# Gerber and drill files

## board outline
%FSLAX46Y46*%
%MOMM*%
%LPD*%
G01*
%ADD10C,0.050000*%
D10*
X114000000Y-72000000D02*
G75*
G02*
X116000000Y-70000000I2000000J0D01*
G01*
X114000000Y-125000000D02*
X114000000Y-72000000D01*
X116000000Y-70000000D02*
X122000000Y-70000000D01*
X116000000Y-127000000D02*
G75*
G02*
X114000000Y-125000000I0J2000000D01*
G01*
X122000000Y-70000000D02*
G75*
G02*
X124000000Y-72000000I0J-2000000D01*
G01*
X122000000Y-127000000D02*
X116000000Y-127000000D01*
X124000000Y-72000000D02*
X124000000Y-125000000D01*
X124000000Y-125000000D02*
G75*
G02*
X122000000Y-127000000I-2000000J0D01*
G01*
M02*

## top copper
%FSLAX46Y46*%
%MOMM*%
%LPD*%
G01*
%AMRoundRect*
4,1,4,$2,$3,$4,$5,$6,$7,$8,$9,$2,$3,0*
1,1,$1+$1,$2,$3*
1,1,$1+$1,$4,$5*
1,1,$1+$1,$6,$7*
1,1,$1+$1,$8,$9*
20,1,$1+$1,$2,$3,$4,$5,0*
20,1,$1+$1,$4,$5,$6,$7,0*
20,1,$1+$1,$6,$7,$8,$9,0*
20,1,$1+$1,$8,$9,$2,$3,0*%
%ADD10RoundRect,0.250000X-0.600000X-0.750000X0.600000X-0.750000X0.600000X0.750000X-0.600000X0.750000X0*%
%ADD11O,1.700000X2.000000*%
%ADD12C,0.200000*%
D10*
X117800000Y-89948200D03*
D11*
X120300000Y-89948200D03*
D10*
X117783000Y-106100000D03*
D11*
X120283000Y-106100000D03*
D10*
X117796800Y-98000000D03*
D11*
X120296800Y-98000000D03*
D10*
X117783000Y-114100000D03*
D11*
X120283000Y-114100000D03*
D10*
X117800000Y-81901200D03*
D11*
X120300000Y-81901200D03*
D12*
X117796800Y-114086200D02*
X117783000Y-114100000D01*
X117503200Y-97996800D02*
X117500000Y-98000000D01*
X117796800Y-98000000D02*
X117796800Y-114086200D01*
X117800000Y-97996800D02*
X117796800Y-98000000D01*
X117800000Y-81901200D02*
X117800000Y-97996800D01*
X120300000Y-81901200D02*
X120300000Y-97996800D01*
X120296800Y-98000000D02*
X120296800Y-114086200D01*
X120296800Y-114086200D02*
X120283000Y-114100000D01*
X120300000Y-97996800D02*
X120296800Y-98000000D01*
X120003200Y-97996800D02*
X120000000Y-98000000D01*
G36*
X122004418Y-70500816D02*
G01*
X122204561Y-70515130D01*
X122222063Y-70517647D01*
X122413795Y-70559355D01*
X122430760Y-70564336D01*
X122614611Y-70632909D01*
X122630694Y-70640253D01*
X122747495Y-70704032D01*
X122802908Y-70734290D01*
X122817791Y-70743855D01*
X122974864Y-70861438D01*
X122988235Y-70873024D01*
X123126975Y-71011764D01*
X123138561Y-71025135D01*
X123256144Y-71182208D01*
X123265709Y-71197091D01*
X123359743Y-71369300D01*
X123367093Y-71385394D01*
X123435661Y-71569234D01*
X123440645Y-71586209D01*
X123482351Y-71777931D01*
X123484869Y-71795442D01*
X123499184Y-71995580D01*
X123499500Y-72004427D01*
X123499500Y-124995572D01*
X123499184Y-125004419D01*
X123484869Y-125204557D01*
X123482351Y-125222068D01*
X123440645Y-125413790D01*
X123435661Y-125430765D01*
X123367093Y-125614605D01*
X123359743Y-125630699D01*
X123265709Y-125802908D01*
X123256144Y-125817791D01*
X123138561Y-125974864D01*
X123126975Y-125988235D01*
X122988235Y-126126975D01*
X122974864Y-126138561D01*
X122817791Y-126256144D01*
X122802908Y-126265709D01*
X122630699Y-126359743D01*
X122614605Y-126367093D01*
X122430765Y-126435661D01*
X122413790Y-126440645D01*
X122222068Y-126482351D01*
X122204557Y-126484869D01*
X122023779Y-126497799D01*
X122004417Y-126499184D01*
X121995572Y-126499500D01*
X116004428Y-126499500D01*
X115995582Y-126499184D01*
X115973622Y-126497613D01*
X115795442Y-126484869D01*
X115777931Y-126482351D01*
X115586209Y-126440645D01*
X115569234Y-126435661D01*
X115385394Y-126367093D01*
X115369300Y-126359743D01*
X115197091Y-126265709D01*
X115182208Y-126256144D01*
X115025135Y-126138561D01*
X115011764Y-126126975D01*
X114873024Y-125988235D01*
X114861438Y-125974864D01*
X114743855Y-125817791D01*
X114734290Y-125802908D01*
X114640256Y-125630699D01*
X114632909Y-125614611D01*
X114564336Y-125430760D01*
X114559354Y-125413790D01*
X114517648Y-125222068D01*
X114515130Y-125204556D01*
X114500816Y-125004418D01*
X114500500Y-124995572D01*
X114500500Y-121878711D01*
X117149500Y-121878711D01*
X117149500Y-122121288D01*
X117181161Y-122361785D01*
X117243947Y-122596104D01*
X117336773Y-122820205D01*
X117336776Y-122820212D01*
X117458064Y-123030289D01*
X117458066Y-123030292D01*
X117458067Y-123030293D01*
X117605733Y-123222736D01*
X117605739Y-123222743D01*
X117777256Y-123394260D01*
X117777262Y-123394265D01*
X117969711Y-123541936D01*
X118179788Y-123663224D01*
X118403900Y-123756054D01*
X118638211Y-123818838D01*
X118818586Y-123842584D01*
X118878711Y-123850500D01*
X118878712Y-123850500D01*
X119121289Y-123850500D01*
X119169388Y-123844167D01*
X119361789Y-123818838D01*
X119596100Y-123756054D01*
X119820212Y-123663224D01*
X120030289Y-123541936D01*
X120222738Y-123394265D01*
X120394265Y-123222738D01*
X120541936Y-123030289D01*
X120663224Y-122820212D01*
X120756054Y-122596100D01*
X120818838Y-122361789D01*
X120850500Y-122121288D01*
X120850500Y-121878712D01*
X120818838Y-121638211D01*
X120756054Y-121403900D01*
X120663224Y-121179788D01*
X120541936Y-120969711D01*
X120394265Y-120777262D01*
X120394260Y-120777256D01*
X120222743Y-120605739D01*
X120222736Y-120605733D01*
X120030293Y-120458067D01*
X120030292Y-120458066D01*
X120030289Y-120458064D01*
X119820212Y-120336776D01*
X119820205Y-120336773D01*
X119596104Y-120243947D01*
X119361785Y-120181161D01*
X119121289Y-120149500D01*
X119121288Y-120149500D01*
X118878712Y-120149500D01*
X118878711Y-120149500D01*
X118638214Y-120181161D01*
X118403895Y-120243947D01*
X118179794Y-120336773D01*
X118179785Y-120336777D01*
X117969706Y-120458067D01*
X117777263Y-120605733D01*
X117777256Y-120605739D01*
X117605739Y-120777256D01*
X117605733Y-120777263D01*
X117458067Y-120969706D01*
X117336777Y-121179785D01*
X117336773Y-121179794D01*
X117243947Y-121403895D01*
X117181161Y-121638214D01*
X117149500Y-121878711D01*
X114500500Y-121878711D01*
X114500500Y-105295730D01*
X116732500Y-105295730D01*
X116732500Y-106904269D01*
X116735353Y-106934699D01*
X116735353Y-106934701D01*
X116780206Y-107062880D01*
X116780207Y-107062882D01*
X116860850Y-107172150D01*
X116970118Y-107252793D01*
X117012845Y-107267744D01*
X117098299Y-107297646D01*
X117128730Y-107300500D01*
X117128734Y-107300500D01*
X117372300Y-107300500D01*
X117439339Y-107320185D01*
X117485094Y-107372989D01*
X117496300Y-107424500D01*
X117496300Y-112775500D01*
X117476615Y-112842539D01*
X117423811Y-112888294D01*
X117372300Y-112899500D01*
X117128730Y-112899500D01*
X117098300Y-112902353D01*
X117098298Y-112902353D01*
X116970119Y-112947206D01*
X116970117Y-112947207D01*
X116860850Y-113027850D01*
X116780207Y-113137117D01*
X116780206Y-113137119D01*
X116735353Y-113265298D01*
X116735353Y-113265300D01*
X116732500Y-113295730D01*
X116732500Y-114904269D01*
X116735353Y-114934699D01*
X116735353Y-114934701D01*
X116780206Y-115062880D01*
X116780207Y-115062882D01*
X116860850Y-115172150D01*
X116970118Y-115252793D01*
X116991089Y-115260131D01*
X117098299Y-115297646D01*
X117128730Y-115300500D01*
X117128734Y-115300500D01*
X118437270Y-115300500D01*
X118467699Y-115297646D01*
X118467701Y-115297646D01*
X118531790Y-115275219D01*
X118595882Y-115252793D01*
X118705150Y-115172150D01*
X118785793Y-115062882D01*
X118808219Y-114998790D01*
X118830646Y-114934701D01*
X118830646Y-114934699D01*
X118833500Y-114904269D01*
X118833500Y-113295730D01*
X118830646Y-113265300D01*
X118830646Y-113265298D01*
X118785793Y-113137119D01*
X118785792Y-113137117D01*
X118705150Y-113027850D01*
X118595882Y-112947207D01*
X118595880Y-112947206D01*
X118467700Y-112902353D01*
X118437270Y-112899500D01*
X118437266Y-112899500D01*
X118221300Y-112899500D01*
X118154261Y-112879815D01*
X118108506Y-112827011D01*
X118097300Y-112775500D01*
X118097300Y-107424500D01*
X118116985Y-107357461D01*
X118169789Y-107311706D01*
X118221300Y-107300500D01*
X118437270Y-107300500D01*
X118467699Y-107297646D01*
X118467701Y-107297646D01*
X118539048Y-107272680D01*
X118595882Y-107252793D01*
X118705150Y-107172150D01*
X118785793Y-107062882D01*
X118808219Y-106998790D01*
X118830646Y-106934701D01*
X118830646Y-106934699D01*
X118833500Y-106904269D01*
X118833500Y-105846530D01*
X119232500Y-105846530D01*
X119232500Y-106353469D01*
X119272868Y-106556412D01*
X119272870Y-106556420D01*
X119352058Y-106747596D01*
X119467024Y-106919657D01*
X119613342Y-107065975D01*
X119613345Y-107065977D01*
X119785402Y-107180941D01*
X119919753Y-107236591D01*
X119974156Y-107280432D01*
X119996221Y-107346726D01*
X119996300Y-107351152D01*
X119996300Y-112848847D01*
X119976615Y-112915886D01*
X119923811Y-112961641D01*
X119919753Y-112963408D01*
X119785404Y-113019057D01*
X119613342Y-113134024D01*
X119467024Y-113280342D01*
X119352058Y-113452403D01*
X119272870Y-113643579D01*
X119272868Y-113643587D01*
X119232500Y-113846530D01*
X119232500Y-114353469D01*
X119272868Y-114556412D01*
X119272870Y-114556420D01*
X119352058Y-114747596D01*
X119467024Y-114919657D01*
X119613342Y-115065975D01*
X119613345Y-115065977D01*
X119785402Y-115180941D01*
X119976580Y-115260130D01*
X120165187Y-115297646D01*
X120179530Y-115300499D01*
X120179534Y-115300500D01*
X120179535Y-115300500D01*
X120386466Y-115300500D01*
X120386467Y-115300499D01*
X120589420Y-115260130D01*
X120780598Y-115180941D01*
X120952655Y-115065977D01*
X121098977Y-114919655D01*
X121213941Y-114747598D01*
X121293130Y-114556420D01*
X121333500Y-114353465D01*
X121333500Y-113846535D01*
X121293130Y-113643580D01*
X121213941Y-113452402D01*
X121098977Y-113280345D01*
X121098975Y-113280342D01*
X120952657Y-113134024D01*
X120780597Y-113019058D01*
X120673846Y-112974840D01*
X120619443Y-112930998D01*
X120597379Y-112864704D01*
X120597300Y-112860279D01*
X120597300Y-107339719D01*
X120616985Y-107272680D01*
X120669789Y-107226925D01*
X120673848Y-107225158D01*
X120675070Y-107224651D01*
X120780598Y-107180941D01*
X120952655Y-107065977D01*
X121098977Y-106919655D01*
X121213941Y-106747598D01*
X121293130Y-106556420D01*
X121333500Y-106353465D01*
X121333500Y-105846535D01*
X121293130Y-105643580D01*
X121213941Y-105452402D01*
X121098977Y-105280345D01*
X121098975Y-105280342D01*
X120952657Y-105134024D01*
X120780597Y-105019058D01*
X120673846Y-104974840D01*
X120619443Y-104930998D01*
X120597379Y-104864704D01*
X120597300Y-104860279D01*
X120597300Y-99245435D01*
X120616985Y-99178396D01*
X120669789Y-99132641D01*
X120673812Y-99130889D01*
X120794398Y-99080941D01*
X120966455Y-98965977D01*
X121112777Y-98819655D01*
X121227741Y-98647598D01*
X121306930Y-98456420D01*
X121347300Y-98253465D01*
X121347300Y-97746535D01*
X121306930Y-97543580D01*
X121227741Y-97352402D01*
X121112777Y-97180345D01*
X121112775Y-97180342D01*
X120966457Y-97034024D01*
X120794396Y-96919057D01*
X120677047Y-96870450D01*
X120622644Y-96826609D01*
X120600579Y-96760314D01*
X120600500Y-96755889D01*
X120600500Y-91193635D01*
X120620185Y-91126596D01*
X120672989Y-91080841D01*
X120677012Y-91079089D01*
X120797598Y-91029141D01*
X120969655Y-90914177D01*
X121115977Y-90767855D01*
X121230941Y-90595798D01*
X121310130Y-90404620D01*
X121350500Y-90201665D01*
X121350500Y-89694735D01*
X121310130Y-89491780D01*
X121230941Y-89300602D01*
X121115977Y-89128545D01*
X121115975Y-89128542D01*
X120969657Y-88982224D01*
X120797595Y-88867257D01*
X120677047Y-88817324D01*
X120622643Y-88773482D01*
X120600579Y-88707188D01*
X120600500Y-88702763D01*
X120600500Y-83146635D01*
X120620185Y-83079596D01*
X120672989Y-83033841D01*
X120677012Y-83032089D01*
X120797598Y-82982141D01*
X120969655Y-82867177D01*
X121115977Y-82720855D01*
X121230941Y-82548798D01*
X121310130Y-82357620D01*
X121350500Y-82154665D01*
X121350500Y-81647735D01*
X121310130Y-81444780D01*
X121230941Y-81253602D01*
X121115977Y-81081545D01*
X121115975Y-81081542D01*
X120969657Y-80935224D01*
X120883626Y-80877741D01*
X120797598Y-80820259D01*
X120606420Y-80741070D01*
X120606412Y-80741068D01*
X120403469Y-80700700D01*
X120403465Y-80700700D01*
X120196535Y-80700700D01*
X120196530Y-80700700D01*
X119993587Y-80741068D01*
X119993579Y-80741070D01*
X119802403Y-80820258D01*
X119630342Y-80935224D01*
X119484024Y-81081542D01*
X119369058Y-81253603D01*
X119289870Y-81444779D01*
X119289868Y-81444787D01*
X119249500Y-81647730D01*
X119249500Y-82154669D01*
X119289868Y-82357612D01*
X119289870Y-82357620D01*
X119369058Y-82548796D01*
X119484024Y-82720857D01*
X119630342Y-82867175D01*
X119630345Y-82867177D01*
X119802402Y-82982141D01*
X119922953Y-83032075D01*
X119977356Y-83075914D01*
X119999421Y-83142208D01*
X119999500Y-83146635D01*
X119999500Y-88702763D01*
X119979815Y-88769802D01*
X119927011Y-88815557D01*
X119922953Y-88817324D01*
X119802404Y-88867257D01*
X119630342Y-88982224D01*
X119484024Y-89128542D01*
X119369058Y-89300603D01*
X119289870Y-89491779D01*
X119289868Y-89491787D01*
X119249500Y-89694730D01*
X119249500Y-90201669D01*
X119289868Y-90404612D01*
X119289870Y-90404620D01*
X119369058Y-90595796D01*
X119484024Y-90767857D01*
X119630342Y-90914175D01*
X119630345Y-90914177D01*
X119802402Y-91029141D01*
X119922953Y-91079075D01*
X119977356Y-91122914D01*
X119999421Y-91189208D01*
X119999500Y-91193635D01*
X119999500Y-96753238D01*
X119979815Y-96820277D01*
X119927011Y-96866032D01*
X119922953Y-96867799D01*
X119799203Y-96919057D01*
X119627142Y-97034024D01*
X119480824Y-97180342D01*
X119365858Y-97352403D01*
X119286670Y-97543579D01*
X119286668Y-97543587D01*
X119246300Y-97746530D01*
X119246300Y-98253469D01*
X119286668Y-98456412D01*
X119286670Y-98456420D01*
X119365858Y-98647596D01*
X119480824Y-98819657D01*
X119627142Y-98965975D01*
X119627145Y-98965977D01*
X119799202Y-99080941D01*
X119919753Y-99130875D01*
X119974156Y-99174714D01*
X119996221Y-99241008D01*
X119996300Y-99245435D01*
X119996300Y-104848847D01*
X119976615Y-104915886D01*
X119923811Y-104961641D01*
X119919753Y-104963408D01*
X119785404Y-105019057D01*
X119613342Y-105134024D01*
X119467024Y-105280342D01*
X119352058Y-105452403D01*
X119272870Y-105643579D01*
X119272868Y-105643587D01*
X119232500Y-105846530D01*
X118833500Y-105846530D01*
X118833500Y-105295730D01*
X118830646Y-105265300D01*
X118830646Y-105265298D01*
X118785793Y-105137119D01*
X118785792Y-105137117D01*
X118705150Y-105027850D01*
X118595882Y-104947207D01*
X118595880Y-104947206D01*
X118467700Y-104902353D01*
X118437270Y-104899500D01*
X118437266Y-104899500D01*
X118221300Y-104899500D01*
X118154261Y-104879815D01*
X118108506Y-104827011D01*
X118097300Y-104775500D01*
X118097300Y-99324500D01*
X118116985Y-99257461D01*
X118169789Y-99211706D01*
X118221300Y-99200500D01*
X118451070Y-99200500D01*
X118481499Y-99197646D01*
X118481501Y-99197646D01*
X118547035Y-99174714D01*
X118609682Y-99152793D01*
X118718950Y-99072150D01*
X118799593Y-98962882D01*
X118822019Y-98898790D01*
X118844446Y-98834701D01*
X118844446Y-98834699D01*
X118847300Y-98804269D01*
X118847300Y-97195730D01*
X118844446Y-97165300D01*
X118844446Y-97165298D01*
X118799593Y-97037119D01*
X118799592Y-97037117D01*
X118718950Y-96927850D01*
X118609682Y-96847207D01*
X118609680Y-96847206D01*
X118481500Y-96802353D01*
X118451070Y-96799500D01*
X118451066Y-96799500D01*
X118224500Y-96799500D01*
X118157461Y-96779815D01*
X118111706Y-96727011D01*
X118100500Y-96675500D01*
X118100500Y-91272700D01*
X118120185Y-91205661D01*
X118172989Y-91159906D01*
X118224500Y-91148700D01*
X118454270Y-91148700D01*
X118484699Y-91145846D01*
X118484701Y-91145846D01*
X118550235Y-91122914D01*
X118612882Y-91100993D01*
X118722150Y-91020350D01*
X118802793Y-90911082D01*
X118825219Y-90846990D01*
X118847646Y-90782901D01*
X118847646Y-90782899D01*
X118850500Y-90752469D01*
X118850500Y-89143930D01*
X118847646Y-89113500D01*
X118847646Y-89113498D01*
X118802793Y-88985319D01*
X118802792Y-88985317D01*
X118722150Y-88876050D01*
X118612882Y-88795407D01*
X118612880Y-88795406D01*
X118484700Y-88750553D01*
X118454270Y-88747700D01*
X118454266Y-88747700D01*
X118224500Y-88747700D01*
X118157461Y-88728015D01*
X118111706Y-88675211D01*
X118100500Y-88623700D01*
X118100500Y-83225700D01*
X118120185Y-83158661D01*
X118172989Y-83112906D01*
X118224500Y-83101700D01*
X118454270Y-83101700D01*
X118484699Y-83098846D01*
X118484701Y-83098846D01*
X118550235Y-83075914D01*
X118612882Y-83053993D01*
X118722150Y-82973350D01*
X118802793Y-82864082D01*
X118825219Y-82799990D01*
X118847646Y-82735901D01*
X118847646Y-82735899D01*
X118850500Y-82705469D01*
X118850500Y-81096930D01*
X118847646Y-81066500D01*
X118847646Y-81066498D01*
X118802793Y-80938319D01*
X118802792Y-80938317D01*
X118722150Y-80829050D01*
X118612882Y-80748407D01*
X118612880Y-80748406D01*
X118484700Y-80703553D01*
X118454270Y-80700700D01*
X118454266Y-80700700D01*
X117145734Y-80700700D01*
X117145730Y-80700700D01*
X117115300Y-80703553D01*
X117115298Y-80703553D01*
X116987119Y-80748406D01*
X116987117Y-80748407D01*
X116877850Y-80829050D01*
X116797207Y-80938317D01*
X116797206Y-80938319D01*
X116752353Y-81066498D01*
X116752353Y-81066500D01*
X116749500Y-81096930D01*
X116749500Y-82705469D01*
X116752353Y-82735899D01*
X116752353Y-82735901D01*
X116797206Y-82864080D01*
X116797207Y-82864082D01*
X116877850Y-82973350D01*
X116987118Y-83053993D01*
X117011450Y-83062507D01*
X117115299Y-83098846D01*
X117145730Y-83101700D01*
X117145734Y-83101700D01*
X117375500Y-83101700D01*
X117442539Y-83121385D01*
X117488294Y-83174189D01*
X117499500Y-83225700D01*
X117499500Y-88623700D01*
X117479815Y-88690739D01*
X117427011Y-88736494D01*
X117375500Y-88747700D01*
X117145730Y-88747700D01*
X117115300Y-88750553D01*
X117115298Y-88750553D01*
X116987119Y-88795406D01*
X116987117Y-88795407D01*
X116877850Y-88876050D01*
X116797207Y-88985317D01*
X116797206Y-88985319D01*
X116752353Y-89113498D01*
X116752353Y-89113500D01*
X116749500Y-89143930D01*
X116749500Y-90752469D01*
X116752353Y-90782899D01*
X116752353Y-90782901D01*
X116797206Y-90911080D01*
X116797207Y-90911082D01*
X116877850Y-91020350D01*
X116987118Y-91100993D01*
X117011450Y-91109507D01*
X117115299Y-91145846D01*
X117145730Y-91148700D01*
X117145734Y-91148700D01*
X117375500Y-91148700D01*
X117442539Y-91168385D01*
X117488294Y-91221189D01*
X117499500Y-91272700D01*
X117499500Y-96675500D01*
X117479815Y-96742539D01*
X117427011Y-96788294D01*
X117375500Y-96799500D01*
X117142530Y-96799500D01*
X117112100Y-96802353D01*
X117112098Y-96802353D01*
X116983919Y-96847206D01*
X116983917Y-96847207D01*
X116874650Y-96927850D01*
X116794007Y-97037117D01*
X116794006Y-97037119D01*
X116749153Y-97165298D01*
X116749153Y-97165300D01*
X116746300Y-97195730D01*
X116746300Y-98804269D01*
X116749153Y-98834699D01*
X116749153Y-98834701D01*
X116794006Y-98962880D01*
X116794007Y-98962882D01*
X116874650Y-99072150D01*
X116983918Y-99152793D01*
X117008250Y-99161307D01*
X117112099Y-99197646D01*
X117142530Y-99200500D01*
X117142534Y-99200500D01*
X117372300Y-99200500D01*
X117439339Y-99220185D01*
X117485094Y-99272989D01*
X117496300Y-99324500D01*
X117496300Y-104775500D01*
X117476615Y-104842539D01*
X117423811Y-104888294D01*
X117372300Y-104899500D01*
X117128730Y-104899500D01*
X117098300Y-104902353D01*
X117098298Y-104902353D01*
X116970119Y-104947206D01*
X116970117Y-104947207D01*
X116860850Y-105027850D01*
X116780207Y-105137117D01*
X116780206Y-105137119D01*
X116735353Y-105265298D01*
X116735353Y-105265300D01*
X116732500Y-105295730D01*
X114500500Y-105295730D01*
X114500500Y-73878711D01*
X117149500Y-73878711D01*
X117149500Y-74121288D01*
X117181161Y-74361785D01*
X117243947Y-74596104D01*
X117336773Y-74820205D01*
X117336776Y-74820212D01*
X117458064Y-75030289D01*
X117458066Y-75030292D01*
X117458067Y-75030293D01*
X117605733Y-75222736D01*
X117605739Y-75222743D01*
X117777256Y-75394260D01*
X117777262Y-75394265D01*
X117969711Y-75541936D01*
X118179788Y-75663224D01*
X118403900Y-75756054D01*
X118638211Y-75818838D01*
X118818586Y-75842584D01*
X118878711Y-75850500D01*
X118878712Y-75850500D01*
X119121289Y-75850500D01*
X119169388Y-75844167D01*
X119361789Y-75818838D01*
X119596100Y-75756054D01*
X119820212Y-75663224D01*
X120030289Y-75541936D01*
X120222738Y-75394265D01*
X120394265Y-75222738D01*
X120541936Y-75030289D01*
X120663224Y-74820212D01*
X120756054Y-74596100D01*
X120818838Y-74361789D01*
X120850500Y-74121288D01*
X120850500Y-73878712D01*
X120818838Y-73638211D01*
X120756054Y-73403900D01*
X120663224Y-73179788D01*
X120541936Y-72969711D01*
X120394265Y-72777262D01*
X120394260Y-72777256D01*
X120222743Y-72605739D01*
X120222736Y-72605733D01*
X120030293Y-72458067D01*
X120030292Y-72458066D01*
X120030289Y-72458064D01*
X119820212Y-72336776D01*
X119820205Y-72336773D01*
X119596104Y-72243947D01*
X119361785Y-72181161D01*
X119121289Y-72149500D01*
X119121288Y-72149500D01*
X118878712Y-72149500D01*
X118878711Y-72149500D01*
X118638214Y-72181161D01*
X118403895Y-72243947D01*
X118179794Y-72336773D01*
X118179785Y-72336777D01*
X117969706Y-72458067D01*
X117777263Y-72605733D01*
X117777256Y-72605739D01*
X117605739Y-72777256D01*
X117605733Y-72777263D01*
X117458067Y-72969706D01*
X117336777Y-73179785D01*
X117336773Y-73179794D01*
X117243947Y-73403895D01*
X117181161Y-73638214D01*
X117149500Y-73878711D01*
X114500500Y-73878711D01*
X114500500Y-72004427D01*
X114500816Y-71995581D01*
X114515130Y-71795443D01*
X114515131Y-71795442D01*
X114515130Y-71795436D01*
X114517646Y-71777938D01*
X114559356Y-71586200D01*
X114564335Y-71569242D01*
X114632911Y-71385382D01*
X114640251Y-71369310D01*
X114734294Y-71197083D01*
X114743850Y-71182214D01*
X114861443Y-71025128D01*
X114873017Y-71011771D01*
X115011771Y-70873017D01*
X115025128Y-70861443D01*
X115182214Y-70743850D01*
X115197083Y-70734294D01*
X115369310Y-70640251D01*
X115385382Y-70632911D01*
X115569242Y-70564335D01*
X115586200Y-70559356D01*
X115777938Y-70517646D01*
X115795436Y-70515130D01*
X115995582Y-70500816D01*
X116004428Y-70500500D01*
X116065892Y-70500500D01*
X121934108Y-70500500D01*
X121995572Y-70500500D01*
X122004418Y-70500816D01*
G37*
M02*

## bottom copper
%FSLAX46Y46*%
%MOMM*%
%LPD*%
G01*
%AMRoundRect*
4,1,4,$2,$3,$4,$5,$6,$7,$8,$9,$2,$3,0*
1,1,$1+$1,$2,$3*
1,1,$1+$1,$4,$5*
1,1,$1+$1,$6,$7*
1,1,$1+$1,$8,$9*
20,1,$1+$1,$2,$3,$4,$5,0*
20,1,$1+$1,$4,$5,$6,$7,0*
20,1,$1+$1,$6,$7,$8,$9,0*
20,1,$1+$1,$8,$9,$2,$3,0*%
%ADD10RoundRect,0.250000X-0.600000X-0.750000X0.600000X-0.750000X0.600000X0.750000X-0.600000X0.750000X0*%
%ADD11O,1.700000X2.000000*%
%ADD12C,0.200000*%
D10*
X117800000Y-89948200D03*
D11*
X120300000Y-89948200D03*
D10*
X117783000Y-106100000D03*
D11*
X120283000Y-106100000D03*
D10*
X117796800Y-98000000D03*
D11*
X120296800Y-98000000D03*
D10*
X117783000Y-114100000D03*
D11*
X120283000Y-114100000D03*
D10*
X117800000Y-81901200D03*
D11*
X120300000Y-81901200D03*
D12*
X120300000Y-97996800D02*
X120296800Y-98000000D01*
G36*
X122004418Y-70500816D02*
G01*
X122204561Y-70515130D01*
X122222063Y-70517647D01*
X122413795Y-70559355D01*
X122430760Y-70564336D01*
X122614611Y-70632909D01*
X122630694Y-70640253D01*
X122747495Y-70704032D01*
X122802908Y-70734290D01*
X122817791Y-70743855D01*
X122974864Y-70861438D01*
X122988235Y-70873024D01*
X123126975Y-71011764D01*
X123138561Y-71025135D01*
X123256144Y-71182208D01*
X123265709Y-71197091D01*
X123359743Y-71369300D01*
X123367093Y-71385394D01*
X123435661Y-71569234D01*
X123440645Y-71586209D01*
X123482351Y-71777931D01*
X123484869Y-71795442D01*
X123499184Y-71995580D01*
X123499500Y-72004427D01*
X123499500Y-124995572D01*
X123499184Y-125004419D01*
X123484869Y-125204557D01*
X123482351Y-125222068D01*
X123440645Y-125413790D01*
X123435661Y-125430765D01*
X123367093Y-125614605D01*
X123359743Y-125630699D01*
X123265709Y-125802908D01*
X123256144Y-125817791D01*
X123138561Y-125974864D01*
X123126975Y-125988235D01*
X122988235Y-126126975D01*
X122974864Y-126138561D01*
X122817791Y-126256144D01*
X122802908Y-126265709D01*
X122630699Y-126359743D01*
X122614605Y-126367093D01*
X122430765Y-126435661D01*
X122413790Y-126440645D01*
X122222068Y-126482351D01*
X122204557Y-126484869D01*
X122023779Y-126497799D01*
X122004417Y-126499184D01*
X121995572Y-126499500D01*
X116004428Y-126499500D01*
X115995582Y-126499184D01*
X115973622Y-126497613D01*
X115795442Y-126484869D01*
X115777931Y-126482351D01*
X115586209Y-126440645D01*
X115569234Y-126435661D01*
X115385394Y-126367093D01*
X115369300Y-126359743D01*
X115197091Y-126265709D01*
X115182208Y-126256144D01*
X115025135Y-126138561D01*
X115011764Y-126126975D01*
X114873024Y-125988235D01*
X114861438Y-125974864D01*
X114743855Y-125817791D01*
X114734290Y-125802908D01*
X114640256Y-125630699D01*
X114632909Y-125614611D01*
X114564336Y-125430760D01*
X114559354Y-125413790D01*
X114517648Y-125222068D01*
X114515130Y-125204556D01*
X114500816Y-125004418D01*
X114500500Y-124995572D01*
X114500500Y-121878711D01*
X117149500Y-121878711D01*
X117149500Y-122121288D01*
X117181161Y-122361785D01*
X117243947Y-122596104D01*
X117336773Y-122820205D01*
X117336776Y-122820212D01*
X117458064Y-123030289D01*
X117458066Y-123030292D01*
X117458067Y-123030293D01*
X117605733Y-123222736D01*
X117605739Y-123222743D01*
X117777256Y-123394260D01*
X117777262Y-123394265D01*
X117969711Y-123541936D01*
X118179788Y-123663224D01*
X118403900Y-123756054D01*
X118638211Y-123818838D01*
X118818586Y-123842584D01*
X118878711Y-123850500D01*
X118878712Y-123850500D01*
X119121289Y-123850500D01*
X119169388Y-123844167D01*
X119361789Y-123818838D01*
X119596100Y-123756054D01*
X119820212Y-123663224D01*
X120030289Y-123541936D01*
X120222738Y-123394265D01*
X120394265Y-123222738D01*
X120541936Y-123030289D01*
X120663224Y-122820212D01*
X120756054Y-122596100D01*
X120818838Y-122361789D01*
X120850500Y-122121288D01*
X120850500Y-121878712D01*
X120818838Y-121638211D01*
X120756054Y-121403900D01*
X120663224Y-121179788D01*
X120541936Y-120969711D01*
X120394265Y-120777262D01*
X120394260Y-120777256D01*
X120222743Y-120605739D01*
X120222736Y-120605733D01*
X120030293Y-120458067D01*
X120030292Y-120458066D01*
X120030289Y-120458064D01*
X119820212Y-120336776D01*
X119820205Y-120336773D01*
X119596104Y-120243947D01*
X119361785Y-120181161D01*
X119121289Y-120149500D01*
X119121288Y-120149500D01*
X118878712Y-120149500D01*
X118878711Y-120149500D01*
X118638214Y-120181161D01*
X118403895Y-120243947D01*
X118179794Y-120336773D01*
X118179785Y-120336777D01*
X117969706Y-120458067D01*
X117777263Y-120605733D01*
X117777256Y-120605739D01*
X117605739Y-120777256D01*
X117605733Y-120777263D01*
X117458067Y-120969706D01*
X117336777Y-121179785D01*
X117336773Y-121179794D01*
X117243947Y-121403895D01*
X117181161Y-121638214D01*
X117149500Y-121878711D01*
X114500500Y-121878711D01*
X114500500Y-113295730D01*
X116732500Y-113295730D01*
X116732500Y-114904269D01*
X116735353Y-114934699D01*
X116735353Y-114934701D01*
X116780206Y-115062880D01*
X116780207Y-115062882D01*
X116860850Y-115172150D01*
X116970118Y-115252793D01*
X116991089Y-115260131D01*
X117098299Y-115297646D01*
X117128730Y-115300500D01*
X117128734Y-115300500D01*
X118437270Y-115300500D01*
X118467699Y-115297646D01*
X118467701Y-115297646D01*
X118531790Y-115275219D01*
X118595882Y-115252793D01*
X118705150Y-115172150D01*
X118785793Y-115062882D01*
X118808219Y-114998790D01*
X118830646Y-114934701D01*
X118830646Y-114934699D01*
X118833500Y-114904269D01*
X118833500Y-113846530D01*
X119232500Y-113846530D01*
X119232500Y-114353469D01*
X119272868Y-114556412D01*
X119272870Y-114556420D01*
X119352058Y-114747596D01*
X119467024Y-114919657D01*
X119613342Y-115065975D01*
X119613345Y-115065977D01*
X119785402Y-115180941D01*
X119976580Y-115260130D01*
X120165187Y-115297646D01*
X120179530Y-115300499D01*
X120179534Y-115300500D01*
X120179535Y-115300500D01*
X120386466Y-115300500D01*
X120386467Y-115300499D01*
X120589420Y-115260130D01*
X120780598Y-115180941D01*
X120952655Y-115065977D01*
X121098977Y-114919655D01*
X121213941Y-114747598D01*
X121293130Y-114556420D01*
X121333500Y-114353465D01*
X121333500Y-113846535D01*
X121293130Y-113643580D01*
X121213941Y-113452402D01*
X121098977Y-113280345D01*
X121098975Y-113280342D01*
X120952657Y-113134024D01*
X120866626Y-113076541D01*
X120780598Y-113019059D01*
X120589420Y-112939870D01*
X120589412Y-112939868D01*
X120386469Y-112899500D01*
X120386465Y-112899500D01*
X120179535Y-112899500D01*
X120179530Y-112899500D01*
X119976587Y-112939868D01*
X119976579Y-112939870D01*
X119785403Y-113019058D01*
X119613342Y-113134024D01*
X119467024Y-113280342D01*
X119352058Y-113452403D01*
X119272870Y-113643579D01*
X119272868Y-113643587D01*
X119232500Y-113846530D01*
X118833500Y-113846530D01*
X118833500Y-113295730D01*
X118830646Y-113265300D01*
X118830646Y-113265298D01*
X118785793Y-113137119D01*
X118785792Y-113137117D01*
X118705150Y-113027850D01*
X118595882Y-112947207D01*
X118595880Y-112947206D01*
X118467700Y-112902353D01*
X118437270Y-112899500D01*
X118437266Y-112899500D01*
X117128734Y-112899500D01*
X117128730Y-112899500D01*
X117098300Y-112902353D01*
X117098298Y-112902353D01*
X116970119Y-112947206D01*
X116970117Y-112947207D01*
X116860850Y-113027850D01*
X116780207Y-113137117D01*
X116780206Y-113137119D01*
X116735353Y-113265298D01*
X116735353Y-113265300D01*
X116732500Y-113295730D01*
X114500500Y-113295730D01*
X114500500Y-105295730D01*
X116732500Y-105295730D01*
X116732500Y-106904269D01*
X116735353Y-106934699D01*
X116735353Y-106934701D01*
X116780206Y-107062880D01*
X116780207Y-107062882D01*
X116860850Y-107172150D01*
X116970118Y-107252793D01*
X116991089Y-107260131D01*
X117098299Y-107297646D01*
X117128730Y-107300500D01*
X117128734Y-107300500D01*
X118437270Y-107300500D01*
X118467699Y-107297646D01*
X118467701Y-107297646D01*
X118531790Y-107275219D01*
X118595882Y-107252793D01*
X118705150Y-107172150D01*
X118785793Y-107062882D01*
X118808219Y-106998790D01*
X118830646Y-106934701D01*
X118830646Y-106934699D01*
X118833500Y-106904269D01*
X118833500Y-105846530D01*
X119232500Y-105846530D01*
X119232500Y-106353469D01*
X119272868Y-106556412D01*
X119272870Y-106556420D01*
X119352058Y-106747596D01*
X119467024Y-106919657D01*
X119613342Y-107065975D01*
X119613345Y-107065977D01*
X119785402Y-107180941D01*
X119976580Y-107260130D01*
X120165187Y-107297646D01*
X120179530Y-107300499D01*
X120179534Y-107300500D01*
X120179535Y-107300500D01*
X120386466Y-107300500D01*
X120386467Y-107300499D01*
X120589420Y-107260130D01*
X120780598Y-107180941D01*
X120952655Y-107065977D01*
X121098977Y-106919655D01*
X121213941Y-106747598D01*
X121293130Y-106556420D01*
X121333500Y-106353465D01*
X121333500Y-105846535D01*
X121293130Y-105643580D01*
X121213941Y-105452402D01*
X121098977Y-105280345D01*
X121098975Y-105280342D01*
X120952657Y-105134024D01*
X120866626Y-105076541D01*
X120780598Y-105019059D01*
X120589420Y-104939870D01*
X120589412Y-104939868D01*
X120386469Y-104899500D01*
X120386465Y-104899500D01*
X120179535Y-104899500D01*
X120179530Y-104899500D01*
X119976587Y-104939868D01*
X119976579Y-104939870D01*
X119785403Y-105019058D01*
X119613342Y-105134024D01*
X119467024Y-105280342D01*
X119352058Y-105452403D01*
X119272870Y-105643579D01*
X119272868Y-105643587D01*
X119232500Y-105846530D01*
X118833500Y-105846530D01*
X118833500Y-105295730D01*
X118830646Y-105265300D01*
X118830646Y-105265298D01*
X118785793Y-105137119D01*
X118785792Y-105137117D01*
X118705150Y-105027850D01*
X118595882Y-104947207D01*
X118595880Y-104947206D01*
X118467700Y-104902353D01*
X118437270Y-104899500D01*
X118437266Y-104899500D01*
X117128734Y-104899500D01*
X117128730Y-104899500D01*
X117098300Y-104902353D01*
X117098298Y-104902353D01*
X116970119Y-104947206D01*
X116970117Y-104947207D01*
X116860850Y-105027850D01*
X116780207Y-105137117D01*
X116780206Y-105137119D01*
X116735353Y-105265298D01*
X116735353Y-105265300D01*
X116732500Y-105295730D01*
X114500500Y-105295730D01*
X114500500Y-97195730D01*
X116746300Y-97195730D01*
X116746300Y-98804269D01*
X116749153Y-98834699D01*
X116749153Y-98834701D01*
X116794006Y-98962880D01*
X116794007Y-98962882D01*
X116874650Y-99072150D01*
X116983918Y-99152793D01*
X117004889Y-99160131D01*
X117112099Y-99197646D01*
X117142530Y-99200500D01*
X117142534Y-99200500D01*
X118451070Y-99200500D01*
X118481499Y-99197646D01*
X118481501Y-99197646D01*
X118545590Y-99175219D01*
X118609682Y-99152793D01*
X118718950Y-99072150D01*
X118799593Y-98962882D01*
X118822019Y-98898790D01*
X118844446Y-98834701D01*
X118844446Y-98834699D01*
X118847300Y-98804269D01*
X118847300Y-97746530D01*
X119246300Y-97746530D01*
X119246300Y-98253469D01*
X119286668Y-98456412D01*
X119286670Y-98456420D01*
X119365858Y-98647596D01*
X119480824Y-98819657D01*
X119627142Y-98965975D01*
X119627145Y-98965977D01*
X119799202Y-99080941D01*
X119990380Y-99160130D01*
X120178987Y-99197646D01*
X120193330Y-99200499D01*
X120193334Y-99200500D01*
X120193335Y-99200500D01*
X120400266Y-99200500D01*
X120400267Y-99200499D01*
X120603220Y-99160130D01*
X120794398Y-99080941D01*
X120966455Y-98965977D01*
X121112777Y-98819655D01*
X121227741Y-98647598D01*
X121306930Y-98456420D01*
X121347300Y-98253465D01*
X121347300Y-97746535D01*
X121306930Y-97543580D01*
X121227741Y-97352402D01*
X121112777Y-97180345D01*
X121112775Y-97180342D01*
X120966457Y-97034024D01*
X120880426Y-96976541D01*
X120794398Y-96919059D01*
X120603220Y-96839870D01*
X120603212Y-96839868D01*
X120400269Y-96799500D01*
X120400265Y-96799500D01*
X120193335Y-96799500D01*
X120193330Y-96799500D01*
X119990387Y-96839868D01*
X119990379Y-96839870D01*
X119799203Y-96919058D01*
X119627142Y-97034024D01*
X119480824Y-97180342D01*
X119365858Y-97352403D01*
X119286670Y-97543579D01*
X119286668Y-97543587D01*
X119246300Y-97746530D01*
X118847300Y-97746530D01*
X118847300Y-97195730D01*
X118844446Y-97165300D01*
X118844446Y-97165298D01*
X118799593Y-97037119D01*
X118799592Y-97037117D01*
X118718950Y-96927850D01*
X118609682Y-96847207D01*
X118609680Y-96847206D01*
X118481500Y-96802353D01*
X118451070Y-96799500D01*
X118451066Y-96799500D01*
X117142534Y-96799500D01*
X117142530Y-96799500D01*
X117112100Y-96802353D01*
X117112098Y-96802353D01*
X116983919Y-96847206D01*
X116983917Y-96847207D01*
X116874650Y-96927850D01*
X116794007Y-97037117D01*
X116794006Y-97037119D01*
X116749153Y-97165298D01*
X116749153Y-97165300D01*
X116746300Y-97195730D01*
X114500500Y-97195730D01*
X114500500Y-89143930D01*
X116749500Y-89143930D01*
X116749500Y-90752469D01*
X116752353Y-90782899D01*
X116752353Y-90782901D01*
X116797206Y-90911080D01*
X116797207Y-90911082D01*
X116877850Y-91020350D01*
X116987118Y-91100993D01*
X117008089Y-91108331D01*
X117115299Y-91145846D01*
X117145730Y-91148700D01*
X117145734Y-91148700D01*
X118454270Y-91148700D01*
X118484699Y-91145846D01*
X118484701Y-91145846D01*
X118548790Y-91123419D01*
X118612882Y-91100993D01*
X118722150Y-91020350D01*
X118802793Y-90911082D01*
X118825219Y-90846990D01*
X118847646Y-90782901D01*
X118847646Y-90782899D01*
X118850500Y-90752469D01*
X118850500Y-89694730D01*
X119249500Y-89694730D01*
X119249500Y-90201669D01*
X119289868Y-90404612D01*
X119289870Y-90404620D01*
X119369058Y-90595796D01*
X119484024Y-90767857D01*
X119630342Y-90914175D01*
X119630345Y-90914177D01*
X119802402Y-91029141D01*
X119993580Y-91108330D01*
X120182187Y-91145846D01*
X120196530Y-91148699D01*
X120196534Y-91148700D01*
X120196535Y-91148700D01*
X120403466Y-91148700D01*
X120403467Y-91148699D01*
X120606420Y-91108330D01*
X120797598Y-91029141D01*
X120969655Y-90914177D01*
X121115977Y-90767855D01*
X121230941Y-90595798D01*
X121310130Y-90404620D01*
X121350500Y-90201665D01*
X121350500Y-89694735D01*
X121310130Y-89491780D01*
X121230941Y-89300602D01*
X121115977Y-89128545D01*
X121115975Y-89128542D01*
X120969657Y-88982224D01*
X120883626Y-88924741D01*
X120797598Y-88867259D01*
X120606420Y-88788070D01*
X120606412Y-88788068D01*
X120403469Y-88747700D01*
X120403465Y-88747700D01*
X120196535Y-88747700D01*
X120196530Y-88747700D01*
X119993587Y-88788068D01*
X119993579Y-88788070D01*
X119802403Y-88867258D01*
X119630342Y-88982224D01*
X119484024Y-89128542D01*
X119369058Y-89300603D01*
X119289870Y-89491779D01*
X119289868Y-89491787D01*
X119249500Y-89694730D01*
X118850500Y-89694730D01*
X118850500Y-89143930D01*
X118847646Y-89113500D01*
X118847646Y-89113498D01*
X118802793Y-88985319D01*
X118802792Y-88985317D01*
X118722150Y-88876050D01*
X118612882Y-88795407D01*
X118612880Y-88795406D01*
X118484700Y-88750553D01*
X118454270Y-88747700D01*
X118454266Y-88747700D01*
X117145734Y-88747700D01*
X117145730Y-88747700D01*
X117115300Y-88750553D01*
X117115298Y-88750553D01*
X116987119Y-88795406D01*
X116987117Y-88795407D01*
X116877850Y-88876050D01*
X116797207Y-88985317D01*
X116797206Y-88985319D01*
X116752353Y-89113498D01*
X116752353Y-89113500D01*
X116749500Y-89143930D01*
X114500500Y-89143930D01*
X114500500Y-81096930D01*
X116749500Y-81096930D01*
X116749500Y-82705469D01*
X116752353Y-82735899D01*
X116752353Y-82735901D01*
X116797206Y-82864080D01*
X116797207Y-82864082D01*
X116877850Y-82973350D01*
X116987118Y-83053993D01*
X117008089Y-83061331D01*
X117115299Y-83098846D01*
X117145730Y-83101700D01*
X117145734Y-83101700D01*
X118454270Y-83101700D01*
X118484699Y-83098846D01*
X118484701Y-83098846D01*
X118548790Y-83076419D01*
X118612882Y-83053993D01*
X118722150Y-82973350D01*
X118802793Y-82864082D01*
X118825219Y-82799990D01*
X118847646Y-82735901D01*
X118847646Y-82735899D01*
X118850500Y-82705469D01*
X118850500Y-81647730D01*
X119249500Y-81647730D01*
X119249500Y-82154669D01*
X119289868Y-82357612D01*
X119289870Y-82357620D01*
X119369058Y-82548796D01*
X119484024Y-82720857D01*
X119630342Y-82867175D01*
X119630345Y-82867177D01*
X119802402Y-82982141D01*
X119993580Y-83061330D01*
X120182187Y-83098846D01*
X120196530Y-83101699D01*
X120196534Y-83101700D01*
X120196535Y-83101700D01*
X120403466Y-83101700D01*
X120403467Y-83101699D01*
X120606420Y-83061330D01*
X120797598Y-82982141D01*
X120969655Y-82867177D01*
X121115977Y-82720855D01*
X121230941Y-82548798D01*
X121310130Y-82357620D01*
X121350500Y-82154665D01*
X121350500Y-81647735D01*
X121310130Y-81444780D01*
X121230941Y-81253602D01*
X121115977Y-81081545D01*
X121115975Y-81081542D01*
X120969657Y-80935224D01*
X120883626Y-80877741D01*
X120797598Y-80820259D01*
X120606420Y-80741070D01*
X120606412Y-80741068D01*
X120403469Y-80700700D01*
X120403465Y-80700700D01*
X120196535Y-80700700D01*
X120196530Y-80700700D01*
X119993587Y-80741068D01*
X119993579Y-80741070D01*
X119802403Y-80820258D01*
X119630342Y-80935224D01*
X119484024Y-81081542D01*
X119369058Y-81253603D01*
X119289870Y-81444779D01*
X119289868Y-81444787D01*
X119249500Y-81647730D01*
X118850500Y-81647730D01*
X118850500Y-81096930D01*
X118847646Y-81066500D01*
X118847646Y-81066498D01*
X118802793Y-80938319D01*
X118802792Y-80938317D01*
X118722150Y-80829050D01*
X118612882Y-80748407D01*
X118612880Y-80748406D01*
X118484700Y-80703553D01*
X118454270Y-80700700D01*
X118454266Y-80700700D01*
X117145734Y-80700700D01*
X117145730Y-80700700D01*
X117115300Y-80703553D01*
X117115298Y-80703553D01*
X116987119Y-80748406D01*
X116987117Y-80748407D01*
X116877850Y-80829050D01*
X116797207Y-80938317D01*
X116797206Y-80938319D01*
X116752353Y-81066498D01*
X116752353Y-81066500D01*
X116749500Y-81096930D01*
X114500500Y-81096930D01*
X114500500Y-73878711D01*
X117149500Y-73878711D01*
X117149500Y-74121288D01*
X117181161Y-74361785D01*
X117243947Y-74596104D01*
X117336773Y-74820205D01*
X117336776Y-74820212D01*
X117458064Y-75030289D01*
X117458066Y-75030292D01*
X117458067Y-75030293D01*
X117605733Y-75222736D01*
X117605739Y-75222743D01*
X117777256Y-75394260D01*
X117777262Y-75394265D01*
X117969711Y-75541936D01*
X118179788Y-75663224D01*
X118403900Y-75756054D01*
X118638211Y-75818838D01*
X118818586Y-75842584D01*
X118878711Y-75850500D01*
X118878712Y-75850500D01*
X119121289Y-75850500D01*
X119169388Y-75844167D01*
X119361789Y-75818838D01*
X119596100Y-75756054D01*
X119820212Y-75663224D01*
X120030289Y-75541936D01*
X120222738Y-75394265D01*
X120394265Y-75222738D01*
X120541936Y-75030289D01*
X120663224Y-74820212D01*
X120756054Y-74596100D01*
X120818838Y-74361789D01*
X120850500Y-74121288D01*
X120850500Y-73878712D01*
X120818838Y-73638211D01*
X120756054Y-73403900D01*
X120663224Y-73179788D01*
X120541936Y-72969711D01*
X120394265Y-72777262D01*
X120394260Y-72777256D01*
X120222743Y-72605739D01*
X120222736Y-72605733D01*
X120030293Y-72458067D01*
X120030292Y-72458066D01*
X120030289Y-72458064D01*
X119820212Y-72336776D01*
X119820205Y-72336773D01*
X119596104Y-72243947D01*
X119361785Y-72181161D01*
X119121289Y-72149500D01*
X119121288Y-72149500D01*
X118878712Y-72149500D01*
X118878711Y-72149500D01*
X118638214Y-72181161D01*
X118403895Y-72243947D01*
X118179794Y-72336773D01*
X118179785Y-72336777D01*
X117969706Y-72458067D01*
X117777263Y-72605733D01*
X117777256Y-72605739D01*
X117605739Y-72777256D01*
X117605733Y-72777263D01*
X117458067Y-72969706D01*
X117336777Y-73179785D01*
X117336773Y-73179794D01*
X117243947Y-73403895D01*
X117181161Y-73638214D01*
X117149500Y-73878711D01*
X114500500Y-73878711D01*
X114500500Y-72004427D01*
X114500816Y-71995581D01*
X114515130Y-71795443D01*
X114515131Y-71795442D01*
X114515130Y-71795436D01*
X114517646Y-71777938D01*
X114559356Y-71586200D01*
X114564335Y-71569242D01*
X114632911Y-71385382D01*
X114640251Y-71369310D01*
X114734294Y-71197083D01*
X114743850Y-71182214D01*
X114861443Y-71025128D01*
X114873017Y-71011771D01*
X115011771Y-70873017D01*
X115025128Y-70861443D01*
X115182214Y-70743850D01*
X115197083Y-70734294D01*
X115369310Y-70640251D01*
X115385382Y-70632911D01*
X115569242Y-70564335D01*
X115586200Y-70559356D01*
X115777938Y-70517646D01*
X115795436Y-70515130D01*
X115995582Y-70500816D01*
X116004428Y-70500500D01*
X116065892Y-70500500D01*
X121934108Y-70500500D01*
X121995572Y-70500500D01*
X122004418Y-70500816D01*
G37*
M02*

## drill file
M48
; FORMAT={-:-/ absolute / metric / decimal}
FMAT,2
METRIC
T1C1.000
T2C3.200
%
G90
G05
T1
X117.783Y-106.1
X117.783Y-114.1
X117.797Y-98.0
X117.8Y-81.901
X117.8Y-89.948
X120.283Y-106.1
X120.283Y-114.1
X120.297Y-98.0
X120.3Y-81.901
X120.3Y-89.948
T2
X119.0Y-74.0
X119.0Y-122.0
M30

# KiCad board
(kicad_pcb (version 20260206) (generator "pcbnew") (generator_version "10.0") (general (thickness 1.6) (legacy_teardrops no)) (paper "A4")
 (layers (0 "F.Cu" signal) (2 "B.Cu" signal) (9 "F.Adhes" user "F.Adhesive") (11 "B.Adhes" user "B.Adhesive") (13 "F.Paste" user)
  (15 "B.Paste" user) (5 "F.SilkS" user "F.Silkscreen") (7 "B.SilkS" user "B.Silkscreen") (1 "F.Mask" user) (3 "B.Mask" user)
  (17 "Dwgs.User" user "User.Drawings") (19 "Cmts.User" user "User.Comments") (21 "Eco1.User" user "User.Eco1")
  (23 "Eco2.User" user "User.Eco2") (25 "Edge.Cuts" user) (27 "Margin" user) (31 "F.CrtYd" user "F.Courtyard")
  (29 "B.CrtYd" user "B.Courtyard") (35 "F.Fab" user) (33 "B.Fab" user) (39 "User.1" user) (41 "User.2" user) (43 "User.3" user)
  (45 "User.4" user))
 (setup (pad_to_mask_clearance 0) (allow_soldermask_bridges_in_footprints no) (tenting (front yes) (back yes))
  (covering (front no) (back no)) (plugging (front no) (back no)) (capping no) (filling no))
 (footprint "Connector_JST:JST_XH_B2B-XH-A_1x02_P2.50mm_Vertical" (layer "F.Cu") (at 117.8 89.9482)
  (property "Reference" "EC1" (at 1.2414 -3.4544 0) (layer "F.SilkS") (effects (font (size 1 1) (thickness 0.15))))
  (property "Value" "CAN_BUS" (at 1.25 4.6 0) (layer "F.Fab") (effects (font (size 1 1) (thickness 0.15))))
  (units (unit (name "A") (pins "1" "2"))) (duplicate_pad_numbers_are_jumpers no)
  (pad "1" thru_hole roundrect (at 0 0) (size 1.7 2) (drill 1) (layers "*.Cu" "*.Mask") (remove_unused_layers no)
   (roundrect_rratio 0.147059) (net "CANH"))
  (pad "2" thru_hole oval (at 2.5 0) (size 1.7 2) (drill 1) (layers "*.Cu" "*.Mask") (remove_unused_layers no) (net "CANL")))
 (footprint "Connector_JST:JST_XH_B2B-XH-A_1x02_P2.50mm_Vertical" (layer "F.Cu") (at 117.783 106.1)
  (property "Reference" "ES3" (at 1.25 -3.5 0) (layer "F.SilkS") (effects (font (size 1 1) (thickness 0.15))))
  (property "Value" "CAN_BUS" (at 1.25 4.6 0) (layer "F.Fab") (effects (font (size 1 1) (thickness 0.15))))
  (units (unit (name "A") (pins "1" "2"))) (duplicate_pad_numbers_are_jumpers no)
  (pad "1" thru_hole roundrect (at 0 0) (size 1.7 2) (drill 1) (layers "*.Cu" "*.Mask") (remove_unused_layers no)
   (roundrect_rratio 0.147059) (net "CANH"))
  (pad "2" thru_hole oval (at 2.5 0) (size 1.7 2) (drill 1) (layers "*.Cu" "*.Mask") (remove_unused_layers no) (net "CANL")))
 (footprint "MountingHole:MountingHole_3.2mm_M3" (layer "F.Cu") (at 119 122)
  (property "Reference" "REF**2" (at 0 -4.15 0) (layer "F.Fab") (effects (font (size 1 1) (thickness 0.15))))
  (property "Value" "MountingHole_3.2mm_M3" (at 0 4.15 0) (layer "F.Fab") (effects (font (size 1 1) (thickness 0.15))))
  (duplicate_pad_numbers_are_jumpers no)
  (pad "" np_thru_hole circle (at 0 0) (size 3.2 3.2) (drill 3.2) (layers "*.Cu" "*.Mask")))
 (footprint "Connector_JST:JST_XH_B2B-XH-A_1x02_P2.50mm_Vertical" (layer "F.Cu") (at 117.7968 98)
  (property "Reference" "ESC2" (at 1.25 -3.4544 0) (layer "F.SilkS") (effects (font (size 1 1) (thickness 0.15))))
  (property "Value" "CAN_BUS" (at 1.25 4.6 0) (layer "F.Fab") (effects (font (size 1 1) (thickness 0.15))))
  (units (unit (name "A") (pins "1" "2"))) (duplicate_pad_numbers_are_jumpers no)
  (pad "1" thru_hole roundrect (at 0 0) (size 1.7 2) (drill 1) (layers "*.Cu" "*.Mask") (remove_unused_layers no)
   (roundrect_rratio 0.147059) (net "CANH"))
  (pad "2" thru_hole oval (at 2.5 0) (size 1.7 2) (drill 1) (layers "*.Cu" "*.Mask") (remove_unused_layers no) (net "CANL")))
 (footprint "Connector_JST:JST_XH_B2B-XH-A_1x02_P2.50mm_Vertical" (layer "F.Cu") (at 117.783 114.1)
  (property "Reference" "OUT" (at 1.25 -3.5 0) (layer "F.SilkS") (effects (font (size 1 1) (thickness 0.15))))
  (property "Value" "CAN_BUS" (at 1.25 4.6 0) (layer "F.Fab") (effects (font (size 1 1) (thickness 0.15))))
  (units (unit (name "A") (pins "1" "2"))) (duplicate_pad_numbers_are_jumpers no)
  (pad "1" thru_hole roundrect (at 0 0) (size 1.7 2) (drill 1) (layers "*.Cu" "*.Mask") (remove_unused_layers no)
   (roundrect_rratio 0.147059) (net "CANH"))
  (pad "2" thru_hole oval (at 2.5 0) (size 1.7 2) (drill 1) (layers "*.Cu" "*.Mask") (remove_unused_layers no) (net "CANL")))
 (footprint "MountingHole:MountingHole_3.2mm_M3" (layer "F.Cu") (at 119 74)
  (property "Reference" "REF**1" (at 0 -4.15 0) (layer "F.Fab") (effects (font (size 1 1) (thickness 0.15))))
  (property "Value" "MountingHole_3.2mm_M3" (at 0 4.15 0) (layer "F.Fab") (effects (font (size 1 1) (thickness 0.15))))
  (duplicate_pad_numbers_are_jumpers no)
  (pad "" np_thru_hole circle (at 0 0) (size 3.2 3.2) (drill 3.2) (layers "*.Cu" "*.Mask")))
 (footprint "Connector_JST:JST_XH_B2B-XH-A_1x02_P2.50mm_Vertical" (layer "F.Cu") (at 117.8 81.9012)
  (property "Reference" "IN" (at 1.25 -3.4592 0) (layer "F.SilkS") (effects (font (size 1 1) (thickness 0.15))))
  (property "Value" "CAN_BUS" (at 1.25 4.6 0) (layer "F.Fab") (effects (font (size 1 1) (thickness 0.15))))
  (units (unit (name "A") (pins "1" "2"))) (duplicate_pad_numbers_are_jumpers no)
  (pad "1" thru_hole roundrect (at 0 0) (size 1.7 2) (drill 1) (layers "*.Cu" "*.Mask") (remove_unused_layers no)
   (roundrect_rratio 0.147059) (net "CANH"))
  (pad "2" thru_hole oval (at 2.5 0) (size 1.7 2) (drill 1) (layers "*.Cu" "*.Mask") (remove_unused_layers no) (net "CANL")))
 (gr_arc (start 114 72) (mid 114.585786 70.585786) (end 116 70) (stroke (width 0.05) (type default)) (layer "Edge.Cuts"))
 (gr_line (start 114 125) (end 114 72) (stroke (width 0.05) (type default)) (layer "Edge.Cuts"))
 (gr_line (start 116 70) (end 122 70) (stroke (width 0.05) (type default)) (layer "Edge.Cuts"))
 (gr_arc (start 116 127) (mid 114.585786 126.414214) (end 114 125) (stroke (width 0.05) (type default)) (layer "Edge.Cuts"))
 (gr_arc (start 122 70) (mid 123.414214 70.585786) (end 124 72) (stroke (width 0.05) (type default)) (layer "Edge.Cuts"))
 (gr_line (start 122 127) (end 116 127) (stroke (width 0.05) (type default)) (layer "Edge.Cuts"))
 (gr_line (start 124 72) (end 124 125) (stroke (width 0.05) (type default)) (layer "Edge.Cuts"))
 (gr_arc (start 124 125) (mid 123.414214 126.414214) (end 122 127) (stroke (width 0.05) (type default)) (layer "Edge.Cuts"))
 (segment (start 117.7968 114.0862) (end 117.783 114.1) (width 0.2) (layer "F.Cu") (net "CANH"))
 (segment (start 117.5032 97.9968) (end 117.5 98) (width 0.2) (layer "F.Cu") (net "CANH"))
 (segment (start 117.7968 98) (end 117.7968 114.0862) (width 0.2) (layer "F.Cu") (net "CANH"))
 (segment (start 117.8 97.9968) (end 117.7968 98) (width 0.2) (layer "F.Cu") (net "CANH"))
 (segment (start 117.8 81.9012) (end 117.8 97.9968) (width 0.2) (layer "F.Cu") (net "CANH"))
 (segment (start 120.3 81.9012) (end 120.3 97.9968) (width 0.2) (layer "F.Cu") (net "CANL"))
 (segment (start 120.2968 98) (end 120.2968 114.0862) (width 0.2) (layer "F.Cu") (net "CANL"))
 (segment (start 120.2968 114.0862) (end 120.283 114.1) (width 0.2) (layer "F.Cu") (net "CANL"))
 (segment (start 120.3 97.9968) (end 120.2968 98) (width 0.2) (layer "F.Cu") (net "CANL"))
 (segment (start 120.0032 97.9968) (end 120 98) (width 0.2) (layer "F.Cu") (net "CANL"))
 (segment (start 120.3 97.9968) (end 120.2968 98) (width 0.2) (layer "B.Cu") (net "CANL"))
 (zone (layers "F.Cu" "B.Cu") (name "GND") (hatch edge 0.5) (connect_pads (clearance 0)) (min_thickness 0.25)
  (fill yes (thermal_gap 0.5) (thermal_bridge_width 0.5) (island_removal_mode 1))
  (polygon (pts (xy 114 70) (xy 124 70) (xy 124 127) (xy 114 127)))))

